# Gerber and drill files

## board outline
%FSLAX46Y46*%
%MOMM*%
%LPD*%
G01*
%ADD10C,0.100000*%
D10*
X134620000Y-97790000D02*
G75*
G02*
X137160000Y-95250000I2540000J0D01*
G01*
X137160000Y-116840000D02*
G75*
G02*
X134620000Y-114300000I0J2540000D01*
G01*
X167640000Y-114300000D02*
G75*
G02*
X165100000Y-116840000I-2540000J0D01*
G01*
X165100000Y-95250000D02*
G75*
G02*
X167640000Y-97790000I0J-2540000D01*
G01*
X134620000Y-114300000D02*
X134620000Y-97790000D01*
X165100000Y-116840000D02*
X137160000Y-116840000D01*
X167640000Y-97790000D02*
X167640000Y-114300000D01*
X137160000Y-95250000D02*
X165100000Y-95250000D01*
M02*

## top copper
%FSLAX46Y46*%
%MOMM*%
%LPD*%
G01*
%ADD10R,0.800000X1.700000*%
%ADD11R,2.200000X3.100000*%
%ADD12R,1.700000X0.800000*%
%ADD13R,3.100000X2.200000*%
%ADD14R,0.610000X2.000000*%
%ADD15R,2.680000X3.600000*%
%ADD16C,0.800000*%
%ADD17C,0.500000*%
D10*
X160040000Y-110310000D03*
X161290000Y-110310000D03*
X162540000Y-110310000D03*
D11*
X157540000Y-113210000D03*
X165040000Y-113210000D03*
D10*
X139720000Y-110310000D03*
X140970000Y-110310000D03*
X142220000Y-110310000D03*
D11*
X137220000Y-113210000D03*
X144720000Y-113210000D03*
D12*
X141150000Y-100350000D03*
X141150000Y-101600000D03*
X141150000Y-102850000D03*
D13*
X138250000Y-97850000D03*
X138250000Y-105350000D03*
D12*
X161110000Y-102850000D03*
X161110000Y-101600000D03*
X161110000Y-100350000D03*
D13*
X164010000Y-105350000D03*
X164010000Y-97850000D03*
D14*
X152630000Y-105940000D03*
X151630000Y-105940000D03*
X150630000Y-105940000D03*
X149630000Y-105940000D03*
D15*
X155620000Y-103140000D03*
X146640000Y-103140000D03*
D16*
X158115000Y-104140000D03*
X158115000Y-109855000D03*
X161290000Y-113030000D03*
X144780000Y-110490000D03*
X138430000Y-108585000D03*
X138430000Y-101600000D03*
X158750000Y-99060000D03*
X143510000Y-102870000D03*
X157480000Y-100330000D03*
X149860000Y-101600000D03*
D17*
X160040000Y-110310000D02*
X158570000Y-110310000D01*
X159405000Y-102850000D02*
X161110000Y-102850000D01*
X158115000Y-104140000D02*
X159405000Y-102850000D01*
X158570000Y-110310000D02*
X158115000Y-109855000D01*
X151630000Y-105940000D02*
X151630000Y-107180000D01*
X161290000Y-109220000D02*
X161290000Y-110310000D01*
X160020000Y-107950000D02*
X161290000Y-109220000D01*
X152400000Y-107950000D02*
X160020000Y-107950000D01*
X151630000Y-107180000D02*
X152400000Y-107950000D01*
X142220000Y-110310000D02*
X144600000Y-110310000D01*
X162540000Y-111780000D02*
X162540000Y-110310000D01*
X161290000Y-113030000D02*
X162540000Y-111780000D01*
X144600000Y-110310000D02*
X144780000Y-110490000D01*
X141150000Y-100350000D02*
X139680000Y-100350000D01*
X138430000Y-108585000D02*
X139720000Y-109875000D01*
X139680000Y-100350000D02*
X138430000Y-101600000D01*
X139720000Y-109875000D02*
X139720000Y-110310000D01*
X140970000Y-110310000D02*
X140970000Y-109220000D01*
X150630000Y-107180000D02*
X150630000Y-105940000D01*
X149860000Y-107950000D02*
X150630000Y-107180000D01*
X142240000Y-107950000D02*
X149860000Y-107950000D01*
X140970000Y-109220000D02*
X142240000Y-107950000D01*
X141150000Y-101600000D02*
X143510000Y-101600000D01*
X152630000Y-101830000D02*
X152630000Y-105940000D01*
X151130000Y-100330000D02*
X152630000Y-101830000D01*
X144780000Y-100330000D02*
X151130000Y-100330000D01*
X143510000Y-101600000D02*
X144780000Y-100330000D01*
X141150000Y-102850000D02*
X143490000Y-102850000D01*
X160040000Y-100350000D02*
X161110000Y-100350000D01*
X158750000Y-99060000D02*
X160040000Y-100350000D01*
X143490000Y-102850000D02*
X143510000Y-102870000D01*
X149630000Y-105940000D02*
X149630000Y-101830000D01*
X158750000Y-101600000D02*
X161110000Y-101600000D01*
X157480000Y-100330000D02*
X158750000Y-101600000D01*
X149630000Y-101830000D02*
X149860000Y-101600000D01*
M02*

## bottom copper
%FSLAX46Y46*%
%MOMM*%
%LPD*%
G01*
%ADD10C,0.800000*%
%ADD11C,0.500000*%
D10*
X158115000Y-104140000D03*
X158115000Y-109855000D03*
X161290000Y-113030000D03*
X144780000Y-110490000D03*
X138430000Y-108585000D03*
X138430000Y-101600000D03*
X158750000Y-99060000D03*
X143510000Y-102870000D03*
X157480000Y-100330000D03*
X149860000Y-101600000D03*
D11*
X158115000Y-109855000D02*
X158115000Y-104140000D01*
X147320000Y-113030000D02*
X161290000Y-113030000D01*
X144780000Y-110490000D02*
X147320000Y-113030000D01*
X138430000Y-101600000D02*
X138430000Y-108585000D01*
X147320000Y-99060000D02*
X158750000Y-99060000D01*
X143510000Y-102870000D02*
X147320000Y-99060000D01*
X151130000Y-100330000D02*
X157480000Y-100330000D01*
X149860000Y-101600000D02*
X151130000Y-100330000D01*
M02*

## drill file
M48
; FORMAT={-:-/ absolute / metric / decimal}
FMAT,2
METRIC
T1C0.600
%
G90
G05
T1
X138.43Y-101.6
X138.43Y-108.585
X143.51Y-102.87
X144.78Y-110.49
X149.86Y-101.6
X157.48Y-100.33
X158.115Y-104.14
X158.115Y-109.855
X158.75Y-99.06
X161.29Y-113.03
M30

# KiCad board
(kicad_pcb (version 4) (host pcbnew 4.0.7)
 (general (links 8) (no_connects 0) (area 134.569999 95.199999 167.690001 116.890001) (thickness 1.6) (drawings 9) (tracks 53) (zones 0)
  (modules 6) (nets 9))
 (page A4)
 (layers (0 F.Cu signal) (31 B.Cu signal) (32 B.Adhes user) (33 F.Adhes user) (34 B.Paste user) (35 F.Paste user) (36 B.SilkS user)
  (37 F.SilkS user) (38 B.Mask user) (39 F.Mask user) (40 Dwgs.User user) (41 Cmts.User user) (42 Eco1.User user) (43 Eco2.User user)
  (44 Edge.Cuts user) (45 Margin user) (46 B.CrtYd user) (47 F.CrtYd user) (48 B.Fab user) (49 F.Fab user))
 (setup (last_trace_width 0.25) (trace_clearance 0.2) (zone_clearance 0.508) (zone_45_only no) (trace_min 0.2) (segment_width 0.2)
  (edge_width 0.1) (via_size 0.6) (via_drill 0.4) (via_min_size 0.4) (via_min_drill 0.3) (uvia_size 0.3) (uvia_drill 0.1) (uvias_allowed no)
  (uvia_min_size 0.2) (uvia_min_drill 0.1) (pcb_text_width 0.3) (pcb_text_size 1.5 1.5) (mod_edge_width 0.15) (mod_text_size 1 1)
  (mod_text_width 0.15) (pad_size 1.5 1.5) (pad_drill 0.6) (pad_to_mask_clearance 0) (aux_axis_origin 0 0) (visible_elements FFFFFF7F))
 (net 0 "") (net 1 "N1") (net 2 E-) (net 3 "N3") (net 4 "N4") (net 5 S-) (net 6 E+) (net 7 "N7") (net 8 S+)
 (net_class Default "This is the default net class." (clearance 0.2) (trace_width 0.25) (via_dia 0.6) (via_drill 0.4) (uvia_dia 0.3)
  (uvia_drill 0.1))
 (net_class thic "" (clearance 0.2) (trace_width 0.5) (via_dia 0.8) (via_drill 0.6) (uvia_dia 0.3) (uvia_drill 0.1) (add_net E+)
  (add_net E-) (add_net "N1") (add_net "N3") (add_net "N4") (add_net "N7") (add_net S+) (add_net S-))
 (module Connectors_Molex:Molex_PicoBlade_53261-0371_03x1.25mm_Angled (layer F.Cu) (at 161.29 111.76)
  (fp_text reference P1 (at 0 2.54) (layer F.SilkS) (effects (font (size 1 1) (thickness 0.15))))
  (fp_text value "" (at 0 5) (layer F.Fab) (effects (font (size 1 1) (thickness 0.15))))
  (pad 1 smd rect (at -1.25 -1.45) (size 0.8 1.7) (layers F.Cu F.Paste F.Mask) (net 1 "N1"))
  (pad 2 smd rect (at 0 -1.45) (size 0.8 1.7) (layers F.Cu F.Paste F.Mask) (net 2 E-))
  (pad 3 smd rect (at 1.25 -1.45) (size 0.8 1.7) (layers F.Cu F.Paste F.Mask) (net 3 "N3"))
  (pad "" smd rect (at -3.75 1.45) (size 2.2 3.1) (layers F.Cu F.Paste F.Mask))
  (pad "" smd rect (at 3.75 1.45) (size 2.2 3.1) (layers F.Cu F.Paste F.Mask)))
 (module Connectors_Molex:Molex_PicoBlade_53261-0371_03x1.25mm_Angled (layer F.Cu) (at 140.97 111.76)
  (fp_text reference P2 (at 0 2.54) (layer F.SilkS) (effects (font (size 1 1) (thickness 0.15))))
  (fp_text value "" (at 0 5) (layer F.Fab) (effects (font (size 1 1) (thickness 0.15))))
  (pad 1 smd rect (at -1.25 -1.45) (size 0.8 1.7) (layers F.Cu F.Paste F.Mask) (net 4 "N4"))
  (pad 2 smd rect (at 0 -1.45) (size 0.8 1.7) (layers F.Cu F.Paste F.Mask) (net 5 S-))
  (pad 3 smd rect (at 1.25 -1.45) (size 0.8 1.7) (layers F.Cu F.Paste F.Mask) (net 3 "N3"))
  (pad "" smd rect (at -3.75 1.45) (size 2.2 3.1) (layers F.Cu F.Paste F.Mask))
  (pad "" smd rect (at 3.75 1.45) (size 2.2 3.1) (layers F.Cu F.Paste F.Mask)))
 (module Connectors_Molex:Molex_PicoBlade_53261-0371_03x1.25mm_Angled (layer F.Cu) (at 139.7 101.6 270)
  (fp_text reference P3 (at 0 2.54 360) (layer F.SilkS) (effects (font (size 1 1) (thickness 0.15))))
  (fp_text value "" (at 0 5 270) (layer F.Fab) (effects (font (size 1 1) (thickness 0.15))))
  (pad 1 smd rect (at -1.25 -1.45 270) (size 0.8 1.7) (layers F.Cu F.Paste F.Mask) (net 4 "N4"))
  (pad 2 smd rect (at 0 -1.45 270) (size 0.8 1.7) (layers F.Cu F.Paste F.Mask) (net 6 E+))
  (pad 3 smd rect (at 1.25 -1.45 270) (size 0.8 1.7) (layers F.Cu F.Paste F.Mask) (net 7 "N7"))
  (pad "" smd rect (at -3.75 1.45 270) (size 2.2 3.1) (layers F.Cu F.Paste F.Mask))
  (pad "" smd rect (at 3.75 1.45 270) (size 2.2 3.1) (layers F.Cu F.Paste F.Mask)))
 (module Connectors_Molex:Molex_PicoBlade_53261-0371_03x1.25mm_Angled (layer F.Cu) (at 162.56 101.6 90)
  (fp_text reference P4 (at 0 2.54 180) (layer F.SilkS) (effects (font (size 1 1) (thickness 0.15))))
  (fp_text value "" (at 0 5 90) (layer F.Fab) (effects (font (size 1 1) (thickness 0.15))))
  (pad 1 smd rect (at -1.25 -1.45 90) (size 0.8 1.7) (layers F.Cu F.Paste F.Mask) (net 1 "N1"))
  (pad 2 smd rect (at 0 -1.45 90) (size 0.8 1.7) (layers F.Cu F.Paste F.Mask) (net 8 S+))
  (pad 3 smd rect (at 1.25 -1.45 90) (size 0.8 1.7) (layers F.Cu F.Paste F.Mask) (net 7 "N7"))
  (pad "" smd rect (at -3.75 1.45 90) (size 2.2 3.1) (layers F.Cu F.Paste F.Mask))
  (pad "" smd rect (at 3.75 1.45 90) (size 2.2 3.1) (layers F.Cu F.Paste F.Mask)))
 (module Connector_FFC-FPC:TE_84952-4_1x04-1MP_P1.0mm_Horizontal (layer F.Cu) (at 151.13 104.14 180)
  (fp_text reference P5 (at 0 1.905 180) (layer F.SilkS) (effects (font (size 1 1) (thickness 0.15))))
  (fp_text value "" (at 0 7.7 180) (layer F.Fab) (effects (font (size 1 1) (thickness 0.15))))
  (pad 1 smd rect (at -1.5 -1.8 180) (size 0.61 2) (layers F.Cu F.Paste F.Mask) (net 6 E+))
  (pad 2 smd rect (at -0.5 -1.8 180) (size 0.61 2) (layers F.Cu F.Paste F.Mask) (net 2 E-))
  (pad 3 smd rect (at 0.5 -1.8 180) (size 0.61 2) (layers F.Cu F.Paste F.Mask) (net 5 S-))
  (pad 4 smd rect (at 1.5 -1.8 180) (size 0.61 2) (layers F.Cu F.Paste F.Mask) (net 8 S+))
  (pad MP smd rect (at -4.49 1 180) (size 2.68 3.6) (layers F.Cu F.Paste F.Mask))
  (pad MP smd rect (at 4.49 1 180) (size 2.68 3.6) (layers F.Cu F.Paste F.Mask)))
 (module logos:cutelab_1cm (layer F.Cu) (at 151.13 111.76)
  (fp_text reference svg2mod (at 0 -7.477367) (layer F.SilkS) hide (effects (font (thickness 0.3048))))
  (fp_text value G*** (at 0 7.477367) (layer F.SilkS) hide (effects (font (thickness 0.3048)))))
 (gr_arc (start 137.16 97.79) (end 134.62 97.79) (angle 90) (layer Edge.Cuts) (width 0.1))
 (gr_arc (start 137.16 114.3) (end 137.16 116.84) (angle 90) (layer Edge.Cuts) (width 0.1))
 (gr_arc (start 165.1 114.3) (end 167.64 114.3) (angle 90) (layer Edge.Cuts) (width 0.1))
 (gr_arc (start 165.1 97.79) (end 165.1 95.25) (angle 90) (layer Edge.Cuts) (width 0.1))
 (gr_line (start 134.62 114.3) (end 134.62 97.79) (angle 90) (layer Edge.Cuts) (width 0.1))
 (gr_line (start 165.1 116.84) (end 137.16 116.84) (angle 90) (layer Edge.Cuts) (width 0.1))
 (gr_line (start 167.64 97.79) (end 167.64 114.3) (angle 90) (layer Edge.Cuts) (width 0.1))
 (gr_line (start 137.16 95.25) (end 165.1 95.25) (angle 90) (layer Edge.Cuts) (width 0.1))
 (segment (start 160.04 110.31) (end 158.57 110.31) (width 0.5) (layer F.Cu) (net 1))
 (segment (start 159.405 102.85) (end 161.11 102.85) (width 0.5) (layer F.Cu) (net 1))
 (segment (start 158.115 104.14) (end 159.405 102.85) (width 0.5) (layer F.Cu) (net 1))
 (via (at 158.115 104.14) (size 0.8) (drill 0.6) (layers F.Cu B.Cu) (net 1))
 (segment (start 158.115 109.855) (end 158.115 104.14) (width 0.5) (layer B.Cu) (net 1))
 (via (at 158.115 109.855) (size 0.8) (drill 0.6) (layers F.Cu B.Cu) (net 1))
 (segment (start 158.57 110.31) (end 158.115 109.855) (width 0.5) (layer F.Cu) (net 1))
 (segment (start 151.63 105.94) (end 151.63 107.18) (width 0.5) (layer F.Cu) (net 2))
 (segment (start 161.29 109.22) (end 161.29 110.31) (width 0.5) (layer F.Cu) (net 2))
 (segment (start 160.02 107.95) (end 161.29 109.22) (width 0.5) (layer F.Cu) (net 2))
 (segment (start 152.4 107.95) (end 160.02 107.95) (width 0.5) (layer F.Cu) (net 2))
 (segment (start 151.63 107.18) (end 152.4 107.95) (width 0.5) (layer F.Cu) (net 2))
 (segment (start 142.22 110.31) (end 144.6 110.31) (width 0.5) (layer F.Cu) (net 3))
 (segment (start 162.54 111.78) (end 162.54 110.31) (width 0.5) (layer F.Cu) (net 3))
 (segment (start 161.29 113.03) (end 162.54 111.78) (width 0.5) (layer F.Cu) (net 3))
 (via (at 161.29 113.03) (size 0.8) (drill 0.6) (layers F.Cu B.Cu) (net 3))
 (segment (start 147.32 113.03) (end 161.29 113.03) (width 0.5) (layer B.Cu) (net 3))
 (segment (start 144.78 110.49) (end 147.32 113.03) (width 0.5) (layer B.Cu) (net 3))
 (via (at 144.78 110.49) (size 0.8) (drill 0.6) (layers F.Cu B.Cu) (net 3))
 (segment (start 144.6 110.31) (end 144.78 110.49) (width 0.5) (layer F.Cu) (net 3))
 (segment (start 141.15 100.35) (end 139.68 100.35) (width 0.5) (layer F.Cu) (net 4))
 (segment (start 138.43 108.585) (end 139.72 109.875) (width 0.5) (layer F.Cu) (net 4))
 (via (at 138.43 108.585) (size 0.8) (drill 0.6) (layers F.Cu B.Cu) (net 4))
 (segment (start 138.43 101.6) (end 138.43 108.585) (width 0.5) (layer B.Cu) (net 4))
 (via (at 138.43 101.6) (size 0.8) (drill 0.6) (layers F.Cu B.Cu) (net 4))
 (segment (start 139.68 100.35) (end 138.43 101.6) (width 0.5) (layer F.Cu) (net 4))
 (segment (start 139.72 109.875) (end 139.72 110.31) (width 0.5) (layer F.Cu) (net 4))
 (segment (start 140.97 110.31) (end 140.97 109.22) (width 0.5) (layer F.Cu) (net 5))
 (segment (start 150.63 107.18) (end 150.63 105.94) (width 0.5) (layer F.Cu) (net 5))
 (segment (start 149.86 107.95) (end 150.63 107.18) (width 0.5) (layer F.Cu) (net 5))
 (segment (start 142.24 107.95) (end 149.86 107.95) (width 0.5) (layer F.Cu) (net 5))
 (segment (start 140.97 109.22) (end 142.24 107.95) (width 0.5) (layer F.Cu) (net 5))
 (segment (start 141.15 101.6) (end 143.51 101.6) (width 0.5) (layer F.Cu) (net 6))
 (segment (start 152.63 101.83) (end 152.63 105.94) (width 0.5) (layer F.Cu) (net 6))
 (segment (start 151.13 100.33) (end 152.63 101.83) (width 0.5) (layer F.Cu) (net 6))
 (segment (start 144.78 100.33) (end 151.13 100.33) (width 0.5) (layer F.Cu) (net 6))
 (segment (start 143.51 101.6) (end 144.78 100.33) (width 0.5) (layer F.Cu) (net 6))
 (segment (start 141.15 102.85) (end 143.49 102.85) (width 0.5) (layer F.Cu) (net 7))
 (segment (start 160.04 100.35) (end 161.11 100.35) (width 0.5) (layer F.Cu) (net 7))
 (segment (start 158.75 99.06) (end 160.04 100.35) (width 0.5) (layer F.Cu) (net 7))
 (via (at 158.75 99.06) (size 0.8) (drill 0.6) (layers F.Cu B.Cu) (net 7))
 (segment (start 147.32 99.06) (end 158.75 99.06) (width 0.5) (layer B.Cu) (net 7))
 (segment (start 143.51 102.87) (end 147.32 99.06) (width 0.5) (layer B.Cu) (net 7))
 (via (at 143.51 102.87) (size 0.8) (drill 0.6) (layers F.Cu B.Cu) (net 7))
 (segment (start 143.49 102.85) (end 143.51 102.87) (width 0.5) (layer F.Cu) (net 7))
 (segment (start 149.63 105.94) (end 149.63 101.83) (width 0.5) (layer F.Cu) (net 8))
 (segment (start 158.75 101.6) (end 161.11 101.6) (width 0.5) (layer F.Cu) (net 8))
 (segment (start 157.48 100.33) (end 158.75 101.6) (width 0.5) (layer F.Cu) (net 8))
 (via (at 157.48 100.33) (size 0.8) (drill 0.6) (layers F.Cu B.Cu) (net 8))
 (segment (start 151.13 100.33) (end 157.48 100.33) (width 0.5) (layer B.Cu) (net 8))
 (segment (start 149.86 101.6) (end 151.13 100.33) (width 0.5) (layer B.Cu) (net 8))
 (via (at 149.86 101.6) (size 0.8) (drill 0.6) (layers F.Cu B.Cu) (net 8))
 (segment (start 149.63 101.83) (end 149.86 101.6) (width 0.5) (layer F.Cu) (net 8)))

